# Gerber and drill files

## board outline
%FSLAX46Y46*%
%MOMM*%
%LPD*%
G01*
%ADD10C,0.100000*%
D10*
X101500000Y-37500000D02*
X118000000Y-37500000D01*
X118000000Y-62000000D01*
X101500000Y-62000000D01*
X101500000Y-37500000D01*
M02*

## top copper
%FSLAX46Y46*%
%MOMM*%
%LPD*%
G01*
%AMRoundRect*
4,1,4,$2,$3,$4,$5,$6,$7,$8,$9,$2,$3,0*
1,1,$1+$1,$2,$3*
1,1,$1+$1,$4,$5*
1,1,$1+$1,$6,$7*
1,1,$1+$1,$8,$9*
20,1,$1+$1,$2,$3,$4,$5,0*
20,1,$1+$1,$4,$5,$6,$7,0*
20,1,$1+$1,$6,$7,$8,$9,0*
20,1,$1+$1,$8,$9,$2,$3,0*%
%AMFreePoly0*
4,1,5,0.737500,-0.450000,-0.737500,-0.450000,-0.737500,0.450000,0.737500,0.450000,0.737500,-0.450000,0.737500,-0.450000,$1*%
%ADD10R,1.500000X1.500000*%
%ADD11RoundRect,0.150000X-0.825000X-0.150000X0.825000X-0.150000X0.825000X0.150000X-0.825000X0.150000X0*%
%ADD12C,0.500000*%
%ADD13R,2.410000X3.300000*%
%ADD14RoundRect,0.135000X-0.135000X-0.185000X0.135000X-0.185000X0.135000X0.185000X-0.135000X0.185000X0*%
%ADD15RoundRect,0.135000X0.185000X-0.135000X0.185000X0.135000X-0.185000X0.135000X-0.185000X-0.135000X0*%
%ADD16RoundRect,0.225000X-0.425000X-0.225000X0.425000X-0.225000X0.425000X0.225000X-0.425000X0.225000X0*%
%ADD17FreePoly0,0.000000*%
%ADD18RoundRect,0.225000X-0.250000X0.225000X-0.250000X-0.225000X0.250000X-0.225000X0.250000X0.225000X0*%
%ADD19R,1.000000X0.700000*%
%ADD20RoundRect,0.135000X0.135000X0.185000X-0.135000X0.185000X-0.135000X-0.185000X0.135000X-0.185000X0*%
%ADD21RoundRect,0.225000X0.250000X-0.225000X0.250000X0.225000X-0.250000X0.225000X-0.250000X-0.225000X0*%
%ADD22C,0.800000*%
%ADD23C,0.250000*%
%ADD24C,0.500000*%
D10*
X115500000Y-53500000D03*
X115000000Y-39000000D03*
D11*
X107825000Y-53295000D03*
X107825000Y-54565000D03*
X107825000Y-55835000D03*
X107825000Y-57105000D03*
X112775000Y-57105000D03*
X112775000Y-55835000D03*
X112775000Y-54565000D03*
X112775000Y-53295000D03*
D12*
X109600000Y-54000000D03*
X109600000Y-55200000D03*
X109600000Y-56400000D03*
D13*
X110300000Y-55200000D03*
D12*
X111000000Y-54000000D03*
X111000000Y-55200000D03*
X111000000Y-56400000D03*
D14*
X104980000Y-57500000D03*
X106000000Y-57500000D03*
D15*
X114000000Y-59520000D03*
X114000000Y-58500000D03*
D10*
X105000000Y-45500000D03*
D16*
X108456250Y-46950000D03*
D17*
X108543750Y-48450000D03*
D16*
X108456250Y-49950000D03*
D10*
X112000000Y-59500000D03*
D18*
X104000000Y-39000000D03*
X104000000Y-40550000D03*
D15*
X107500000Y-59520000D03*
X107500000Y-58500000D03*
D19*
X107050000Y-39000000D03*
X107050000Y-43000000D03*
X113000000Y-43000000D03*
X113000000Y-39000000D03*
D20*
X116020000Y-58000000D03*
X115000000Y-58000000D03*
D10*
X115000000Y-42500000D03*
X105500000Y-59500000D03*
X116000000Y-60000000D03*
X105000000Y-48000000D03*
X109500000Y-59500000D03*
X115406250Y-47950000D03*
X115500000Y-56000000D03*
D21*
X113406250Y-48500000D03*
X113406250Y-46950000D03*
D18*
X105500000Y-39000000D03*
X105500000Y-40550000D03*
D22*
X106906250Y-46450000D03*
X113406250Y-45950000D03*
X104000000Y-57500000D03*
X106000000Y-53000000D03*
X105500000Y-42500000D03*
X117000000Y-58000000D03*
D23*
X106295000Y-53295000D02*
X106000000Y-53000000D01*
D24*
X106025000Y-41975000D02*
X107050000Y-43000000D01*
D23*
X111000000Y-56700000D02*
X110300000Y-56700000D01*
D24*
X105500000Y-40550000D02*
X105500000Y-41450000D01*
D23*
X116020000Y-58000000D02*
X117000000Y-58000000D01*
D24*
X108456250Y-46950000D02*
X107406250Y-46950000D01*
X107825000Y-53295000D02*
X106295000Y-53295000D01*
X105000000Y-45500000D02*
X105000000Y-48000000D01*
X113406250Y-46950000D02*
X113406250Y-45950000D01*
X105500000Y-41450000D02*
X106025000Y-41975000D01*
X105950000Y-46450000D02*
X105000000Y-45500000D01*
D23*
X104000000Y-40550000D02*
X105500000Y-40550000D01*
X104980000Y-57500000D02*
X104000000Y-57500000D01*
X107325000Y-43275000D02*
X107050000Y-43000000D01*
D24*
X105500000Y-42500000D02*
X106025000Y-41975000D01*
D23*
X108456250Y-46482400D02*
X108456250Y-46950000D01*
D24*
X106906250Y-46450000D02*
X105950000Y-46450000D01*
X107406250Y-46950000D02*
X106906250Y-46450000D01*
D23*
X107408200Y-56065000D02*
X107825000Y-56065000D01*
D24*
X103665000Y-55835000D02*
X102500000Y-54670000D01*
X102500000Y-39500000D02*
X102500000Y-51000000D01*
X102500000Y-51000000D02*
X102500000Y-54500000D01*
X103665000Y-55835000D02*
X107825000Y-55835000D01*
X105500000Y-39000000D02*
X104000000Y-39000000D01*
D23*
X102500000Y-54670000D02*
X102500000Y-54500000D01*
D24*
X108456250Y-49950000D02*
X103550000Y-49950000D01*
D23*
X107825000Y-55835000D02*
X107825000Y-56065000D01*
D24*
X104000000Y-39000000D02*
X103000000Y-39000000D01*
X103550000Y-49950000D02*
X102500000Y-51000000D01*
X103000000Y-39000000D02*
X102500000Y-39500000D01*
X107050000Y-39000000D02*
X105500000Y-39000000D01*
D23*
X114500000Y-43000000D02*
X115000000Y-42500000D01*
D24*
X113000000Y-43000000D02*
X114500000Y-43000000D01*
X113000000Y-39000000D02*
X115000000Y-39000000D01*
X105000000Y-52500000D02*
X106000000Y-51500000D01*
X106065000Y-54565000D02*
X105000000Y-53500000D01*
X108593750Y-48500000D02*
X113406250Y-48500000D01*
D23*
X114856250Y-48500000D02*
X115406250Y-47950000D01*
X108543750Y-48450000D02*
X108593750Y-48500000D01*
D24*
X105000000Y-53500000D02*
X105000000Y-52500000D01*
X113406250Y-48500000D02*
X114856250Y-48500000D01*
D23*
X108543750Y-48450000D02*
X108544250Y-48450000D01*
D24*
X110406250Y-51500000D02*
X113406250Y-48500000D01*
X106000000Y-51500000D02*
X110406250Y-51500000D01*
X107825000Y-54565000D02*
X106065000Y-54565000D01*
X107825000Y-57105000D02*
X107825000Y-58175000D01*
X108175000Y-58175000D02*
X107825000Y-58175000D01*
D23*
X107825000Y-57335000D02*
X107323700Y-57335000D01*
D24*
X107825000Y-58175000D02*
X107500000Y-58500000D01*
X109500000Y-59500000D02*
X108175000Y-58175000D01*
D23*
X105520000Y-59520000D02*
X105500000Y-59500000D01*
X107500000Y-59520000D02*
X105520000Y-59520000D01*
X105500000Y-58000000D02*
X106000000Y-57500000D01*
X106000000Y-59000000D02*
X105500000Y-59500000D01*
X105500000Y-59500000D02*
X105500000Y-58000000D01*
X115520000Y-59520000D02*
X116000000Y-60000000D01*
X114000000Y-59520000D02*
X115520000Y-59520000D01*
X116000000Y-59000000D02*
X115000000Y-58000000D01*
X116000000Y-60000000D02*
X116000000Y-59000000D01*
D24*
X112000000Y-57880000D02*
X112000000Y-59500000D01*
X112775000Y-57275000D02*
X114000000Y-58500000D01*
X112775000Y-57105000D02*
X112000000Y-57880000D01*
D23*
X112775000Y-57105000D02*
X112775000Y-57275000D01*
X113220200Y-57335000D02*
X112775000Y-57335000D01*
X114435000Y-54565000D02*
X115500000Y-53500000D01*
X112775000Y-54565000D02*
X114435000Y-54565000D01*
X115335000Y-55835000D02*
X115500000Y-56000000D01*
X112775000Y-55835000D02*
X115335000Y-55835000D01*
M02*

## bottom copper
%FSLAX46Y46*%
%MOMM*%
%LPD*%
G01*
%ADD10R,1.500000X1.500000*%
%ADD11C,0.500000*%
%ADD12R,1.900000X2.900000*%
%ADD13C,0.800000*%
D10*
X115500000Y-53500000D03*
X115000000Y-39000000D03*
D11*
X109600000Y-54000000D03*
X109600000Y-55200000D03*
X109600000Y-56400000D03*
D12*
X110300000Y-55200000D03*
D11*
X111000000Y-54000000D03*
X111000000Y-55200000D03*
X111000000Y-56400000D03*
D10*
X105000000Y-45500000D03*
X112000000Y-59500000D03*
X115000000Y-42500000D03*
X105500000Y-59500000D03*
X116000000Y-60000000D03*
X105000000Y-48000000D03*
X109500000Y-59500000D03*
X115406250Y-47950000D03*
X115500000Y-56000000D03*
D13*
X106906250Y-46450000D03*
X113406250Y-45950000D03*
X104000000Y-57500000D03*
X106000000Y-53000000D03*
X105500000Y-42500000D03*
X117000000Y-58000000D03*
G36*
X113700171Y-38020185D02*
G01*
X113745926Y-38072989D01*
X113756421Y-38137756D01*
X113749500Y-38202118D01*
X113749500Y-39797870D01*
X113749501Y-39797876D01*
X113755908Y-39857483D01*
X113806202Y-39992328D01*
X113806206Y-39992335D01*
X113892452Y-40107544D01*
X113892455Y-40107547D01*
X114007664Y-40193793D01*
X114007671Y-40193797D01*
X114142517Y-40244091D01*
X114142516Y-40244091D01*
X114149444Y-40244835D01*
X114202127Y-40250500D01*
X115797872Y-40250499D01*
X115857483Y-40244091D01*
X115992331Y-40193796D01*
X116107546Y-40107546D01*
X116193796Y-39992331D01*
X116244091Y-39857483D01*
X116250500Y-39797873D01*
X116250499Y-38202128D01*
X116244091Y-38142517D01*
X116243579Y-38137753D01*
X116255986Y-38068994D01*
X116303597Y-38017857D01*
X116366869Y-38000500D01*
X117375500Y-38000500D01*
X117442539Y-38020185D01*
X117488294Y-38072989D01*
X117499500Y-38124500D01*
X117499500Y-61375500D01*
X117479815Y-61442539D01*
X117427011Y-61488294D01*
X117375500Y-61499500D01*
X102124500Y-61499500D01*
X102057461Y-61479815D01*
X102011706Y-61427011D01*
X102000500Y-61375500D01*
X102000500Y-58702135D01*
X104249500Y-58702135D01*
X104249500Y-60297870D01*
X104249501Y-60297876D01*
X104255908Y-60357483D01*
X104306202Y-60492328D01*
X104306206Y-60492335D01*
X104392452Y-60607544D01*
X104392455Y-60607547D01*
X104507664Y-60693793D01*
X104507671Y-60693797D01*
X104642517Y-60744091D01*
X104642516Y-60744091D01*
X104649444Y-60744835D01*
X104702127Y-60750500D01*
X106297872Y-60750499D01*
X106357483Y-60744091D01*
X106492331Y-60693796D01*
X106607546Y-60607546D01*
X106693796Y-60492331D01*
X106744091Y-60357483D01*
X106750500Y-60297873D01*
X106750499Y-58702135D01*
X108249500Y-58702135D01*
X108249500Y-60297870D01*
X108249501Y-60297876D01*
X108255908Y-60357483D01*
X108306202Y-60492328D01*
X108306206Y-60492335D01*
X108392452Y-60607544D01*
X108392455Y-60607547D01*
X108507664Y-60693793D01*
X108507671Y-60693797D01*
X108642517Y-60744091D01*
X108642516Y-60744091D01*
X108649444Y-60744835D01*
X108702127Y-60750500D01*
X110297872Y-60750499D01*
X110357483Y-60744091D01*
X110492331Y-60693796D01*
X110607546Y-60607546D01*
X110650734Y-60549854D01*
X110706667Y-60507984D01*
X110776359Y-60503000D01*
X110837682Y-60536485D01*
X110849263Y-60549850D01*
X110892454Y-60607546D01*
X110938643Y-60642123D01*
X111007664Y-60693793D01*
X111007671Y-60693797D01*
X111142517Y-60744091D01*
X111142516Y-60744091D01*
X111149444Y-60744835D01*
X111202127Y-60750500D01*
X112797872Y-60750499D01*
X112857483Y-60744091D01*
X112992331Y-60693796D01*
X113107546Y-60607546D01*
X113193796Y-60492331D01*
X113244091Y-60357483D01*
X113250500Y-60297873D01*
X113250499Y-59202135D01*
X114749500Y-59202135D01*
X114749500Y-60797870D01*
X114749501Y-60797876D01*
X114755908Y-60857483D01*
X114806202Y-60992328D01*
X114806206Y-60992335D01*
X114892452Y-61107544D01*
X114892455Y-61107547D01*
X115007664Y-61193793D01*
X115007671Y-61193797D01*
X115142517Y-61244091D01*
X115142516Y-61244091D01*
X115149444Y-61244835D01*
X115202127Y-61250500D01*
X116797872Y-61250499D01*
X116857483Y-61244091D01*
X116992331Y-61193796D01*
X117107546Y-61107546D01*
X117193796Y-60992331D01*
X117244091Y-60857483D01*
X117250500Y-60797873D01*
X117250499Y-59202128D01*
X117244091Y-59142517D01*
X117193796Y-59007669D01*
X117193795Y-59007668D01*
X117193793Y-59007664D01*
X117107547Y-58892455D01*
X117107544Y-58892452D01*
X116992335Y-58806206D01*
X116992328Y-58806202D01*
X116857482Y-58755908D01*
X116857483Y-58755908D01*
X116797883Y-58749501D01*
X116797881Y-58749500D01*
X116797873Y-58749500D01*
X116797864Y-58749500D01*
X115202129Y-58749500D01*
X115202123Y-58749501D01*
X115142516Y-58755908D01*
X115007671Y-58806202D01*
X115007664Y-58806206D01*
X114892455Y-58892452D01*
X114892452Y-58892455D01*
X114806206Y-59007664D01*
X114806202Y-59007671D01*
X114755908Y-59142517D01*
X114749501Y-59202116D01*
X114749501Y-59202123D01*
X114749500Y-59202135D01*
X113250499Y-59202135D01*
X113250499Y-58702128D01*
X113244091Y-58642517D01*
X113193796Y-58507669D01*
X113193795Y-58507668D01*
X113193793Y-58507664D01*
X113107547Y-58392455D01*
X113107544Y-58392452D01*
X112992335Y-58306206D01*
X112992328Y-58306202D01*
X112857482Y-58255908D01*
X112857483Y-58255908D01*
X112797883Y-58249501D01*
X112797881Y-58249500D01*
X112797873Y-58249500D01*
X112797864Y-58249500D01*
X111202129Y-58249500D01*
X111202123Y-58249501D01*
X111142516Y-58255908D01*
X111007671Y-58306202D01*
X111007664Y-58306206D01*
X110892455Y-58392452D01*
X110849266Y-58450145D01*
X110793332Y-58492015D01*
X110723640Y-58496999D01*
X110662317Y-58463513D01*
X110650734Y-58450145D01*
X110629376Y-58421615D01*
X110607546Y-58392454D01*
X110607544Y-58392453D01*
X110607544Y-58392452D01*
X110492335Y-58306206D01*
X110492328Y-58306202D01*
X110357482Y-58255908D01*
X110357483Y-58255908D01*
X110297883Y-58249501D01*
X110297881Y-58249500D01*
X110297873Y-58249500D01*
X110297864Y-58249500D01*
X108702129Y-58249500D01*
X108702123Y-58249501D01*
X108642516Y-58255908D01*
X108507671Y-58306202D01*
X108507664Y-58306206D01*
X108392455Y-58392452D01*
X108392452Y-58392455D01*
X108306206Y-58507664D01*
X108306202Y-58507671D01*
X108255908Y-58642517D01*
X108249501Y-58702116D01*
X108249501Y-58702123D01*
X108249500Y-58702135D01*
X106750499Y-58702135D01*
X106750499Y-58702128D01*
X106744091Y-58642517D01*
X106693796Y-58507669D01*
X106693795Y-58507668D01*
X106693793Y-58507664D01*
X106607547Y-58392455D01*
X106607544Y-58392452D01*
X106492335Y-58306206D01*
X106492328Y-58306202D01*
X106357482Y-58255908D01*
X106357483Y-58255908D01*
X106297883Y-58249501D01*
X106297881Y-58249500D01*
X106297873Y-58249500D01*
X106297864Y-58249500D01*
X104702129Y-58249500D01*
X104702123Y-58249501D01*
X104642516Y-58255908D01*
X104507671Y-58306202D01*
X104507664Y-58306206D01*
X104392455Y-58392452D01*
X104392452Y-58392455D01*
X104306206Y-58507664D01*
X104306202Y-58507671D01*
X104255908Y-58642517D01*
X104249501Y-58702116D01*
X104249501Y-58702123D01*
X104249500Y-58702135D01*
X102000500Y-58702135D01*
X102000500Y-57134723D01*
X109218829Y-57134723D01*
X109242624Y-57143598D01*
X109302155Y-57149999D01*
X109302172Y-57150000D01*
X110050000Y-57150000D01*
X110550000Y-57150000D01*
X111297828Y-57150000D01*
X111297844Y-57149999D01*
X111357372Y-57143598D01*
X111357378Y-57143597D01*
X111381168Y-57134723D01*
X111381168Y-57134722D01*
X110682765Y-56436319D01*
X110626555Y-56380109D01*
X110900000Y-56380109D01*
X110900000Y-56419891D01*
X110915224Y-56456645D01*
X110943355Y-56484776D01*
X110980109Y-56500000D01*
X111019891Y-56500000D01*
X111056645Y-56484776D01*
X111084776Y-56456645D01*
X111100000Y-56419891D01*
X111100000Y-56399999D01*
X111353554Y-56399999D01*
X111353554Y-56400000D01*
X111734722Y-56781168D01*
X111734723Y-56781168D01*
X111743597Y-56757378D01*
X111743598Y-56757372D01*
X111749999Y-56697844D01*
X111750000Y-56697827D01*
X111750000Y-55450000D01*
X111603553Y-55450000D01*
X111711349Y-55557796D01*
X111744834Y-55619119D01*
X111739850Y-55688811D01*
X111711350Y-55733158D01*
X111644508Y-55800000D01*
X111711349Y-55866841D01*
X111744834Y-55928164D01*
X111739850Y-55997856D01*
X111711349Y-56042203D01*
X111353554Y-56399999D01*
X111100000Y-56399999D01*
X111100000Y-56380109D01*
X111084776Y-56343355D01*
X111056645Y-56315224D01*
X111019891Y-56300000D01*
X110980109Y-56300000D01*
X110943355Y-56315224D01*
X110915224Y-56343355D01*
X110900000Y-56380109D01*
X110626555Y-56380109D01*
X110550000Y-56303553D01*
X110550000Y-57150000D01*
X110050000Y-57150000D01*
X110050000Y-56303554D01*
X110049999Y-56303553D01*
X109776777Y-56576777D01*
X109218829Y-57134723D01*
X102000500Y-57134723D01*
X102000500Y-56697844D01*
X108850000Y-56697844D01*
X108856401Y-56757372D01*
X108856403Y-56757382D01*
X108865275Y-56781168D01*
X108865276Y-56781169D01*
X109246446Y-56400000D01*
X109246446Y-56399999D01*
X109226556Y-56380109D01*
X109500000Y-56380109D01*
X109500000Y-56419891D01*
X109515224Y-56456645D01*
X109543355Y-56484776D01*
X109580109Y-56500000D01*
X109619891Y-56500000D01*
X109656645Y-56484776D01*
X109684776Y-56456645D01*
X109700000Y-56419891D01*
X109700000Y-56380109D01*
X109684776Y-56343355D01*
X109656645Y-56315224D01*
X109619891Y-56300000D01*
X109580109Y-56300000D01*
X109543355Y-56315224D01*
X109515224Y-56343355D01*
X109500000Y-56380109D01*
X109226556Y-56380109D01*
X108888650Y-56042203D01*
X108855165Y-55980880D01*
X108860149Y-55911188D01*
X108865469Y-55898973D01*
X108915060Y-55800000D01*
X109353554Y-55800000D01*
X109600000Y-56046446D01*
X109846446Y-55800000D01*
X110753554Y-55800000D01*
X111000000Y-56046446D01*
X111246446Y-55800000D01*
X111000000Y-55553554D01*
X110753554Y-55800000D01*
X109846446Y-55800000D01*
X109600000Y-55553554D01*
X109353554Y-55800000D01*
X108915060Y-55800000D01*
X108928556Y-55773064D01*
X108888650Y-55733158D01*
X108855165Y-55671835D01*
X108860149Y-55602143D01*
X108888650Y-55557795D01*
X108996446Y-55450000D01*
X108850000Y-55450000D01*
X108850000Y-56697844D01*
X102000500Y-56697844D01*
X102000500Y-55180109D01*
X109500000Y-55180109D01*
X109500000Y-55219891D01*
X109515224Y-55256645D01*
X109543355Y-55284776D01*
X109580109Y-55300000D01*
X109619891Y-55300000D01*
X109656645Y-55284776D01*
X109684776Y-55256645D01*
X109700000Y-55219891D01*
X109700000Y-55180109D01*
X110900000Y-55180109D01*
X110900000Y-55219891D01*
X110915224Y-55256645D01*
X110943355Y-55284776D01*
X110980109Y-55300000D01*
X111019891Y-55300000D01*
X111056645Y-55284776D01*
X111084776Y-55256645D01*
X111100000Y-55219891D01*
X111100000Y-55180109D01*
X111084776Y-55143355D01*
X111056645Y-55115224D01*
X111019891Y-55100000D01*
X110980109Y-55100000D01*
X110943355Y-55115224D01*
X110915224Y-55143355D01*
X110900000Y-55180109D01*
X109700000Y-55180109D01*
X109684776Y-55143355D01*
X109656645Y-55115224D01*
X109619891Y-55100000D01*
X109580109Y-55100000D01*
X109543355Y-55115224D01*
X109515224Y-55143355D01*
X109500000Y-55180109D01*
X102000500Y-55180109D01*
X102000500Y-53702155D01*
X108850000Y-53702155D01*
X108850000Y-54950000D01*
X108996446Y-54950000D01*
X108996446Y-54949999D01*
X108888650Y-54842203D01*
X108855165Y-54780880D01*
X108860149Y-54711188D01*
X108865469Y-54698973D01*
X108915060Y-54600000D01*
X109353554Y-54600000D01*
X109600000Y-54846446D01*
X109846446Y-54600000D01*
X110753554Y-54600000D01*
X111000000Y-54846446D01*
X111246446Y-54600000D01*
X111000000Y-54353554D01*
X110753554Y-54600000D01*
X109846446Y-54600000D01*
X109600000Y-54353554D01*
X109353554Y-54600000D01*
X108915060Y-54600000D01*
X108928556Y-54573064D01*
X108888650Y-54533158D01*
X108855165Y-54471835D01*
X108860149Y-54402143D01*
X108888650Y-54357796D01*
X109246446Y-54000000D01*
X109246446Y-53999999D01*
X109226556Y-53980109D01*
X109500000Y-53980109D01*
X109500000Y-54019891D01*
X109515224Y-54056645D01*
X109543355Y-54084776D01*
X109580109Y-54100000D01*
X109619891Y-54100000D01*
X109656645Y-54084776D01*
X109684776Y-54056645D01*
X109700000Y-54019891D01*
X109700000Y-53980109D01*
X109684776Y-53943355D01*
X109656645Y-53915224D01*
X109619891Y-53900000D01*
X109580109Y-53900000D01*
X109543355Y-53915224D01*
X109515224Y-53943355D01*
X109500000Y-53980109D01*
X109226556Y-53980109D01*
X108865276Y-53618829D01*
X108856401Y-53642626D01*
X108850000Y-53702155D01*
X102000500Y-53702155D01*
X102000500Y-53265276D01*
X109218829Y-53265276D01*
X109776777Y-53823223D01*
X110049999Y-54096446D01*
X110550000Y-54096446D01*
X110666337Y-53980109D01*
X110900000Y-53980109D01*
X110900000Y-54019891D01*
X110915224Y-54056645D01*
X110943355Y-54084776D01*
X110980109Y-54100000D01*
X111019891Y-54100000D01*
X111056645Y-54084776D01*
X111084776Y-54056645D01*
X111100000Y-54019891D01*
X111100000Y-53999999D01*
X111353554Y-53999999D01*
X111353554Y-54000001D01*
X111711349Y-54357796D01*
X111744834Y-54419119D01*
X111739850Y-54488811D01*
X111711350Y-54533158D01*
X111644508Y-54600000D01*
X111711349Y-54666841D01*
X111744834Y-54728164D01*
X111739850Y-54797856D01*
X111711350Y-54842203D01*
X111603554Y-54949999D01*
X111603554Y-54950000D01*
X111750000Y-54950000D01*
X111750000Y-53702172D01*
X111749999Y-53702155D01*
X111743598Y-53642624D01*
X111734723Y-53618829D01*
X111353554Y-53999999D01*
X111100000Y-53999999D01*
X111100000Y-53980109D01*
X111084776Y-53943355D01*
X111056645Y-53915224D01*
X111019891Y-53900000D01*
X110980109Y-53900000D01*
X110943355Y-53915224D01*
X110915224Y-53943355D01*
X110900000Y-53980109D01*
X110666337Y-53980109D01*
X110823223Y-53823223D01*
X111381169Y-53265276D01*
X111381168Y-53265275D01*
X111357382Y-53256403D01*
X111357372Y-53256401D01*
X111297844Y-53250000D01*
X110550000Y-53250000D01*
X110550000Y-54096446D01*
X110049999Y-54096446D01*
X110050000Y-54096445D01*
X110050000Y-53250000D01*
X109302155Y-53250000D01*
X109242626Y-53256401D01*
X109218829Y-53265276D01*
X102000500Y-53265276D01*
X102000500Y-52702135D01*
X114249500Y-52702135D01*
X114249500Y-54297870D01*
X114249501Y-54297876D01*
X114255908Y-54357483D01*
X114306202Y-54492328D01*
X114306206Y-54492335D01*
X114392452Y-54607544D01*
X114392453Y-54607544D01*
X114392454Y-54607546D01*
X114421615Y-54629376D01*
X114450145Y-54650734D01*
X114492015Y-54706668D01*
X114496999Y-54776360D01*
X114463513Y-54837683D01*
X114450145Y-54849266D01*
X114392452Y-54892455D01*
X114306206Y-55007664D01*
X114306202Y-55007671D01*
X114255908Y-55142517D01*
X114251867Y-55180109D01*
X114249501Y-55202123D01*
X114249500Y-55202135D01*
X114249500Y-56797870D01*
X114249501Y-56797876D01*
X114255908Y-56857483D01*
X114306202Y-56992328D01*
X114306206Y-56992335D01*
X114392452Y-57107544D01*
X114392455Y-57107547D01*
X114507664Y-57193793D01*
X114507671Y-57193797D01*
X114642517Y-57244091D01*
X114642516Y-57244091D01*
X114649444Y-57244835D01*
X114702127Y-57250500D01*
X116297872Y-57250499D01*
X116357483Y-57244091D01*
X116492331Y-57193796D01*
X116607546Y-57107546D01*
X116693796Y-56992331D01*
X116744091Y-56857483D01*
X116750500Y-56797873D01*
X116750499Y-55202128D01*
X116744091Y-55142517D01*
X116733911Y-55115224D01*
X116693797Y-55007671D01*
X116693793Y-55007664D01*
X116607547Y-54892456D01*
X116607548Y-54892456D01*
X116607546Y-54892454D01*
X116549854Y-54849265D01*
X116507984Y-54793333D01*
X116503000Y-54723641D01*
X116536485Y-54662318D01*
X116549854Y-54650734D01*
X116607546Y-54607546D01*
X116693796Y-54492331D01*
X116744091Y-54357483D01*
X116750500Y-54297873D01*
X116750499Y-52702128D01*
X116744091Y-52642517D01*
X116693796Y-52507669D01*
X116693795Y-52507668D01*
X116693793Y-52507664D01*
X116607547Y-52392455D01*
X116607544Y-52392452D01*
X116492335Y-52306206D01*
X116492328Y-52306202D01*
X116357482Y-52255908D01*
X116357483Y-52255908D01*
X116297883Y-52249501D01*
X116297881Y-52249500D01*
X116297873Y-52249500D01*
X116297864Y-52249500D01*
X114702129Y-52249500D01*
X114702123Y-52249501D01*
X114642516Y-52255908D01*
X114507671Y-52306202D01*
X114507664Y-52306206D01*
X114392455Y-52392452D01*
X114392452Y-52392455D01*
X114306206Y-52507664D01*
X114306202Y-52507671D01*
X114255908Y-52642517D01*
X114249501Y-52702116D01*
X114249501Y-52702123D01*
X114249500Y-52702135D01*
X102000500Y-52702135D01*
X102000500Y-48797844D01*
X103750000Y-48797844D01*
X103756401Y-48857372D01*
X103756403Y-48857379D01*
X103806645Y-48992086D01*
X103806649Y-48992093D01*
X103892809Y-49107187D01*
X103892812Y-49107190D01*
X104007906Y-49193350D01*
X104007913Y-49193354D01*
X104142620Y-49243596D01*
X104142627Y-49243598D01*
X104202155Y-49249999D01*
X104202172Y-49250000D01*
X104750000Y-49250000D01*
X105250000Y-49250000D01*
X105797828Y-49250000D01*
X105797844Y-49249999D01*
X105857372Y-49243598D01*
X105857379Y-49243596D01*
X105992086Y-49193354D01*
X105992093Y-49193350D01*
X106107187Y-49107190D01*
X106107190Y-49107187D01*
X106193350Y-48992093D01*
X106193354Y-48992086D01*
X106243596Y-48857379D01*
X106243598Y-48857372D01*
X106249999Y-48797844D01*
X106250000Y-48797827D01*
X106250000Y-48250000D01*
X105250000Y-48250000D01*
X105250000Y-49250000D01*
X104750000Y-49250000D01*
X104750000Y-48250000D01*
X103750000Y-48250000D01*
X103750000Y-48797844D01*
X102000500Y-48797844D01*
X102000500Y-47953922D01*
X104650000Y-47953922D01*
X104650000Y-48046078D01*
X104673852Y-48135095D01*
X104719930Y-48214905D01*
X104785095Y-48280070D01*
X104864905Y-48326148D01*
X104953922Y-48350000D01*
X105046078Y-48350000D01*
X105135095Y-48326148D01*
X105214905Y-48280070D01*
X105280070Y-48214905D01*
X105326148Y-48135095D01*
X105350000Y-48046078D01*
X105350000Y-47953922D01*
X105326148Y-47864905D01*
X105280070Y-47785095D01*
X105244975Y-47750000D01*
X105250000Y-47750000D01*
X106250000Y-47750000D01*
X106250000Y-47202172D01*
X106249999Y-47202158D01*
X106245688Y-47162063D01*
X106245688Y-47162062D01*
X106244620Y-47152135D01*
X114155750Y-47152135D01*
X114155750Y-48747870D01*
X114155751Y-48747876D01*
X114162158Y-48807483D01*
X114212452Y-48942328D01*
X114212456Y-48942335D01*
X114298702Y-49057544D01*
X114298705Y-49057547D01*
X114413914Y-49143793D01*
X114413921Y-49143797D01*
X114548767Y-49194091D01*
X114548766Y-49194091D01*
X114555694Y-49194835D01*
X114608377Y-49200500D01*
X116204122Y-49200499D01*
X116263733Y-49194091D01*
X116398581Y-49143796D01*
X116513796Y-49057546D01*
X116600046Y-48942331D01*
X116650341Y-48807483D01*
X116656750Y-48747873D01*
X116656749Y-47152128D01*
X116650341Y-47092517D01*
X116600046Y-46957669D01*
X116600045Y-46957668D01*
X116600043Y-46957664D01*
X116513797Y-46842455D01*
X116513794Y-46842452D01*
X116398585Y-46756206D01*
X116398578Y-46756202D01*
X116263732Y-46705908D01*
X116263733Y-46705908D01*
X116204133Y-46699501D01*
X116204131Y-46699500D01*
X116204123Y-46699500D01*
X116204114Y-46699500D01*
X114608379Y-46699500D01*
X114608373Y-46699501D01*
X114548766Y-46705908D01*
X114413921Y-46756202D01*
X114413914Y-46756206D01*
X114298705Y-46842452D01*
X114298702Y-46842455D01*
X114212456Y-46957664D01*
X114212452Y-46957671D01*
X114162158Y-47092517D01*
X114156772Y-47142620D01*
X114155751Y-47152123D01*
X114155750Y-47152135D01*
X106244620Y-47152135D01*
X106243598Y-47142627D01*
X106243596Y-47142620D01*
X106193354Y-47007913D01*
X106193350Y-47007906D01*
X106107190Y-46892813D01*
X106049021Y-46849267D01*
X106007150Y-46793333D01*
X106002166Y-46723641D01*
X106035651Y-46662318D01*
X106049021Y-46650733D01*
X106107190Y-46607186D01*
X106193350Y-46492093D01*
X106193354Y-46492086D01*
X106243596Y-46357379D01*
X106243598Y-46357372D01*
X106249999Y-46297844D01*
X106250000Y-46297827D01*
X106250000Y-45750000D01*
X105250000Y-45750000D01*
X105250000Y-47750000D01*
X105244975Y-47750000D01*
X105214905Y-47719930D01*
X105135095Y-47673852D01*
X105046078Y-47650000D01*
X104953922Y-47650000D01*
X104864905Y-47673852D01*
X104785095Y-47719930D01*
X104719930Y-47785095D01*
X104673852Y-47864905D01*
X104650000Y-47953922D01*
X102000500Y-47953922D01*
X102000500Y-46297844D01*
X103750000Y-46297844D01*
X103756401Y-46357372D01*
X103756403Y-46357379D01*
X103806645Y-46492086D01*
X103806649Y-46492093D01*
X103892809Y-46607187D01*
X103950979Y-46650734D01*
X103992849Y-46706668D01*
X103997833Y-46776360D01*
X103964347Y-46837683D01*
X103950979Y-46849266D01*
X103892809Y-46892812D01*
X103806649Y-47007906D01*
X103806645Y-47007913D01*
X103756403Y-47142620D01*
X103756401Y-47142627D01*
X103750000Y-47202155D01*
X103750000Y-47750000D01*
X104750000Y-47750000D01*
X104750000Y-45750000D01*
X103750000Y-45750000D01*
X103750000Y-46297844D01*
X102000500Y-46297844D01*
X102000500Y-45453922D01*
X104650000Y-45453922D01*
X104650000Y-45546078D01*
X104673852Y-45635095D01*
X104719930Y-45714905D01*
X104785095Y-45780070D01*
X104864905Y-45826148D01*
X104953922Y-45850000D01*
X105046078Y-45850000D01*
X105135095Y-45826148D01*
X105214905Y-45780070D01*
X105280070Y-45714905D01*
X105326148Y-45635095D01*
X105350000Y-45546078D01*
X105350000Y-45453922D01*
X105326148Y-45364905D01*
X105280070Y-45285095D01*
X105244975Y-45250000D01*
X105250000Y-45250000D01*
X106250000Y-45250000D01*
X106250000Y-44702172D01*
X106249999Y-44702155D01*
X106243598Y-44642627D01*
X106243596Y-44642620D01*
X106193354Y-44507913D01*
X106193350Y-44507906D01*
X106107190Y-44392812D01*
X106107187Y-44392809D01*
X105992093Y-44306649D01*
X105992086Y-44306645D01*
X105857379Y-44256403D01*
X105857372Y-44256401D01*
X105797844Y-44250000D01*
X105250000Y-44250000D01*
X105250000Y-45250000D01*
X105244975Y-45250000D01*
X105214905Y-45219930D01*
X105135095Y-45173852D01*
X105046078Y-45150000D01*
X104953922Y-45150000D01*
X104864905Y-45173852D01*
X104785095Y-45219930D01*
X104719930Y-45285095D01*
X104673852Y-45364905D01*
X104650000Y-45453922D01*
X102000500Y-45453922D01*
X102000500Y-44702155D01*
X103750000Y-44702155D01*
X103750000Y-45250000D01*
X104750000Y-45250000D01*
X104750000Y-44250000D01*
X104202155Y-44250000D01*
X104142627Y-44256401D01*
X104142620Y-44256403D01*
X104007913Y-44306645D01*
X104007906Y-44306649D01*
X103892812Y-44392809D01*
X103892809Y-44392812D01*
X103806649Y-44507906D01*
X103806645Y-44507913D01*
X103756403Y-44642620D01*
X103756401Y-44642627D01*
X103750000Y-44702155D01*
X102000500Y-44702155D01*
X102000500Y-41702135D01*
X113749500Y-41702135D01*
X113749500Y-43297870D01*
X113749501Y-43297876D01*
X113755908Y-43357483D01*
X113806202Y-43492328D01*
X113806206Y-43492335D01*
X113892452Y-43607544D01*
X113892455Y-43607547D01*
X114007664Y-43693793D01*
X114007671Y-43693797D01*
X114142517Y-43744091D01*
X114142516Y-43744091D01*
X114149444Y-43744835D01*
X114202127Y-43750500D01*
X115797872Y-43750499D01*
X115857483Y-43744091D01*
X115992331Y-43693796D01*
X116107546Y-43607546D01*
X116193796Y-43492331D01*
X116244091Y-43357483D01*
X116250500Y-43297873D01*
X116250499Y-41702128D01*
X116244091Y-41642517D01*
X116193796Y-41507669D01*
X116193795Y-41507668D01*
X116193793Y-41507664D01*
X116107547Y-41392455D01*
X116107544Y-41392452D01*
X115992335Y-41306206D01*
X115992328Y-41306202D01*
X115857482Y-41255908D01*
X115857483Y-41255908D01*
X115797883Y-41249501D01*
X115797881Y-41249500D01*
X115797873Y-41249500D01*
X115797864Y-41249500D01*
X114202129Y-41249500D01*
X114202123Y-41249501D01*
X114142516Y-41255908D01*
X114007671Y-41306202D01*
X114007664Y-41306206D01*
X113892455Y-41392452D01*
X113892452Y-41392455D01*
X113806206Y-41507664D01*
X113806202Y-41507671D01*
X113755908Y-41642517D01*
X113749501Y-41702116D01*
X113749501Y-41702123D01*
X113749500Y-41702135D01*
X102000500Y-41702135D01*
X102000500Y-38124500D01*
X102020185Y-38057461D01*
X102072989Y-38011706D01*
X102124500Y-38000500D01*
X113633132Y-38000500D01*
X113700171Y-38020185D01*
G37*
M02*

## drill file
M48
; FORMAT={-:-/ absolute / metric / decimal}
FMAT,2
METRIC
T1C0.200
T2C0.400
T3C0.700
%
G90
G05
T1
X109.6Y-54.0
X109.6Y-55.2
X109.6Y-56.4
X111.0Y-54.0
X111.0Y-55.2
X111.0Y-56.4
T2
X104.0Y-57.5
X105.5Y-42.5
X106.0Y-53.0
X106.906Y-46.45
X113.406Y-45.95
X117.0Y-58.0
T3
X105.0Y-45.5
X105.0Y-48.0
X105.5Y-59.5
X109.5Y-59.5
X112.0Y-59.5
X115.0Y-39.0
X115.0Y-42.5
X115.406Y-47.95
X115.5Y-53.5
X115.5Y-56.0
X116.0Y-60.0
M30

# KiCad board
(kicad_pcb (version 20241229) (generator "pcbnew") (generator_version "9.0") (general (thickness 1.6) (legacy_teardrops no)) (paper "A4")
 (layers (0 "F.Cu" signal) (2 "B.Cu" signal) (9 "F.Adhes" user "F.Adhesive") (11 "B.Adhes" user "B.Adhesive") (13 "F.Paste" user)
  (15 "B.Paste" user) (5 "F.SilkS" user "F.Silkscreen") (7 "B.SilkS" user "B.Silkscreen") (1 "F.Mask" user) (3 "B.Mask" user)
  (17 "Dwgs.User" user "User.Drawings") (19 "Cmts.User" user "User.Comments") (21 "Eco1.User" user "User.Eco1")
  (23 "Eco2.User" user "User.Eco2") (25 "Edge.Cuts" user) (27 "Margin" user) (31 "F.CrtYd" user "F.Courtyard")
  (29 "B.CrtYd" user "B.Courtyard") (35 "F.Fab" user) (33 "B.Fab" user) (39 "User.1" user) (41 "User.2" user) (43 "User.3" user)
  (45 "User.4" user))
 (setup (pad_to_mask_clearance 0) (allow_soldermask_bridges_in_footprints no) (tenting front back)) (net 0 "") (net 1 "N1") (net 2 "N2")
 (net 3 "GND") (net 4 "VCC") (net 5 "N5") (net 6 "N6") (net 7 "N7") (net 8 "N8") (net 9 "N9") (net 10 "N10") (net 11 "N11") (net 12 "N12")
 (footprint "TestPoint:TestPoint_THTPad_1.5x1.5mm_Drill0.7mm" (layer "F.Cu") (at 115.5 53.5)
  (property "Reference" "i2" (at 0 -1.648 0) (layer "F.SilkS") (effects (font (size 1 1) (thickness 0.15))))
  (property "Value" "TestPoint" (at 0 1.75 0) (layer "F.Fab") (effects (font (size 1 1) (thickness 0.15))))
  (pad "1" thru_hole rect (at 0 0) (size 1.5 1.5) (drill 0.7) (layers "*.Cu" "*.Mask") (remove_unused_layers no) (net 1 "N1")))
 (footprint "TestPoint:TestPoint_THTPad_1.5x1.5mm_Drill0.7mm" (layer "F.Cu") (at 115 39)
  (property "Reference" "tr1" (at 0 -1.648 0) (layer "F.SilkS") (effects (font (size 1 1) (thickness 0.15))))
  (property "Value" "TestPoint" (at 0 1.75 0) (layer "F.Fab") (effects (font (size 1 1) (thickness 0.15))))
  (pad "1" thru_hole rect (at 0 0) (size 1.5 1.5) (drill 0.7) (layers "*.Cu" "*.Mask") (remove_unused_layers no) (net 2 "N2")))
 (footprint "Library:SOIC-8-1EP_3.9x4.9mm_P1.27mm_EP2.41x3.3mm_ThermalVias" (layer "F.Cu") (at 110.3 55.2)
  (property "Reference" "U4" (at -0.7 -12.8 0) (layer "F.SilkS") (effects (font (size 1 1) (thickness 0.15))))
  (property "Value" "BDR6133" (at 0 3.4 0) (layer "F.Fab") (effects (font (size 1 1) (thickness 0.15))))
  (pad "" smd roundrect (at -0.6 -0.825) (size 1.01 1.38) (layers "F.Paste") (roundrect_rratio 0.247525))
  (pad "" smd roundrect (at -0.6 0.825) (size 1.01 1.38) (layers "F.Paste") (roundrect_rratio 0.247525))
  (pad "" smd roundrect (at 0.6 -0.825) (size 1.01 1.38) (layers "F.Paste") (roundrect_rratio 0.247525))
  (pad "" smd roundrect (at 0.6 0.825) (size 1.01 1.38) (layers "F.Paste") (roundrect_rratio 0.247525))
  (pad "1" smd roundrect (at -2.475 -1.905) (size 1.95 0.6) (layers "F.Cu" "F.Mask" "F.Paste") (roundrect_rratio 0.25) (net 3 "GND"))
  (pad "2" smd roundrect (at -2.475 -0.635) (size 1.95 0.6) (layers "F.Cu" "F.Mask" "F.Paste") (roundrect_rratio 0.25) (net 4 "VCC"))
  (pad "3" smd roundrect (at -2.475 0.635) (size 1.95 0.6) (layers "F.Cu" "F.Mask" "F.Paste") (roundrect_rratio 0.25) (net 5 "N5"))
  (pad "4" smd roundrect (at -2.475 1.905) (size 1.95 0.6) (layers "F.Cu" "F.Mask" "F.Paste") (roundrect_rratio 0.25) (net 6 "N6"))
  (pad "5" smd roundrect (at 2.475 1.905) (size 1.95 0.6) (layers "F.Cu" "F.Mask" "F.Paste") (roundrect_rratio 0.25) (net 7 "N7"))
  (pad "6" smd roundrect (at 2.475 0.635) (size 1.95 0.6) (layers "F.Cu" "F.Mask" "F.Paste") (roundrect_rratio 0.25) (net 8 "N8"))
  (pad "7" smd roundrect (at 2.475 -0.635) (size 1.95 0.6) (layers "F.Cu" "F.Mask" "F.Paste") (roundrect_rratio 0.25) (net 1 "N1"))
  (pad "8" smd roundrect (at 2.475 -1.905) (size 1.95 0.6) (layers "F.Cu" "F.Mask" "F.Paste") (roundrect_rratio 0.25) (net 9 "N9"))
  (pad "9" thru_hole circle (at -0.7 -1.2) (size 0.5 0.5) (drill 0.2) (layers "*.Cu") (remove_unused_layers no) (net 3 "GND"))
  (pad "9" thru_hole circle (at -0.7 0) (size 0.5 0.5) (drill 0.2) (layers "*.Cu") (remove_unused_layers no) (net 3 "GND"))
  (pad "9" thru_hole circle (at -0.7 1.2) (size 0.5 0.5) (drill 0.2) (layers "*.Cu") (remove_unused_layers no) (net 3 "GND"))
  (pad "9" smd rect (at 0 0) (size 1.9 2.9) (layers "B.Cu") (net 3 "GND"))
  (pad "9" smd rect (at 0 0) (size 2.41 3.3) (layers "F.Cu" "F.Mask") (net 3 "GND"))
  (pad "9" thru_hole circle (at 0.7 -1.2) (size 0.5 0.5) (drill 0.2) (layers "*.Cu") (remove_unused_layers no) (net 3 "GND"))
  (pad "9" thru_hole circle (at 0.7 0) (size 0.5 0.5) (drill 0.2) (layers "*.Cu") (remove_unused_layers no) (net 3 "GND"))
  (pad "9" thru_hole circle (at 0.7 1.2) (size 0.5 0.5) (drill 0.2) (layers "*.Cu") (remove_unused_layers no) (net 3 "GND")))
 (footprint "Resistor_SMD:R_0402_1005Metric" (layer "F.Cu") (at 105.49 57.5)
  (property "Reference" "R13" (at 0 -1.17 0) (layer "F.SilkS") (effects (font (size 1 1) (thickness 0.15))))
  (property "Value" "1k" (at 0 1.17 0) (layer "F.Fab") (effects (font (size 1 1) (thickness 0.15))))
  (pad "1" smd roundrect (at -0.51 0) (size 0.54 0.64) (layers "F.Cu" "F.Mask" "F.Paste") (roundrect_rratio 0.25) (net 3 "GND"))
  (pad "2" smd roundrect (at 0.51 0) (size 0.54 0.64) (layers "F.Cu" "F.Mask" "F.Paste") (roundrect_rratio 0.25) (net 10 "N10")))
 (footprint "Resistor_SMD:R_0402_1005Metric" (layer "F.Cu") (at 114 59.01 90)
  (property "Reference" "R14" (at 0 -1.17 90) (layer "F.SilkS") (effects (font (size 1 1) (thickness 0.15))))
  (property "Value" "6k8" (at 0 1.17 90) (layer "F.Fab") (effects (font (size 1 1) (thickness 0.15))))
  (pad "1" smd roundrect (at -0.51 0 90) (size 0.54 0.64) (layers "F.Cu" "F.Mask" "F.Paste") (roundrect_rratio 0.25) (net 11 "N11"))
  (pad "2" smd roundrect (at 0.51 0 90) (size 0.54 0.64) (layers "F.Cu" "F.Mask" "F.Paste") (roundrect_rratio 0.25) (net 7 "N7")))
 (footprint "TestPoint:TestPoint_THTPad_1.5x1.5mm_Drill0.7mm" (layer "F.Cu") (at 105 45.5)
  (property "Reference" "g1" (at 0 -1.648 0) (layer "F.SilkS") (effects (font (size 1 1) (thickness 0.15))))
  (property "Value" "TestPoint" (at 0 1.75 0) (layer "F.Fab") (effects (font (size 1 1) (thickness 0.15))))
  (pad "1" thru_hole rect (at 0 0) (size 1.5 1.5) (drill 0.7) (layers "*.Cu" "*.Mask") (remove_unused_layers no) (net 3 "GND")))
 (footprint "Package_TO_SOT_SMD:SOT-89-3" (layer "F.Cu") (at 110.40625 48.45)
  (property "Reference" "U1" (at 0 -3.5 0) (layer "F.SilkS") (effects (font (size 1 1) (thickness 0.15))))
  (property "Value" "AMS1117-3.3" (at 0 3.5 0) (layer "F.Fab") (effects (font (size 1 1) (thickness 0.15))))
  (pad "1" smd roundrect (at -1.95 -1.5) (size 1.3 0.9) (layers "F.Cu" "F.Mask" "F.Paste") (roundrect_rratio 0.25) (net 3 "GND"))
  (pad "2" smd custom (at -1.8625 0) (size 1.475 0.9) (layers "F.Cu" "F.Mask" "F.Paste") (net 4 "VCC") (zone_connect 2)
   (thermal_bridge_angle 45) (options (clearance outline) (anchor rect)) (primitives))
  (pad "3" smd roundrect (at -1.95 1.5) (size 1.3 0.9) (layers "F.Cu" "F.Mask" "F.Paste") (roundrect_rratio 0.25) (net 5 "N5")))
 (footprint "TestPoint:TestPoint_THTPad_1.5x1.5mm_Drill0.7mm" (layer "F.Cu") (at 112 59.5)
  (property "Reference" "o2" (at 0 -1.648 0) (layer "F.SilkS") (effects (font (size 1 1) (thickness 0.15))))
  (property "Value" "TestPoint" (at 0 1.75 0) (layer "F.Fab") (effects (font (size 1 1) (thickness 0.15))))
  (pad "1" thru_hole rect (at 0 0) (size 1.5 1.5) (drill 0.7) (layers "*.Cu" "*.Mask") (remove_unused_layers no) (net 7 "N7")))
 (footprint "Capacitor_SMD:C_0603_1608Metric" (layer "F.Cu") (at 104 39.775 -90)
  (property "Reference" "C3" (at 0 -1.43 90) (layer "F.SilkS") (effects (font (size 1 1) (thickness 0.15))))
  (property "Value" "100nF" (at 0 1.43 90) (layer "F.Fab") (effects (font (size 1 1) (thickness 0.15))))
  (pad "1" smd roundrect (at -0.775 0 270) (size 0.9 0.95) (layers "F.Cu" "F.Mask" "F.Paste") (roundrect_rratio 0.25) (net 5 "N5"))
  (pad "2" smd roundrect (at 0.775 0 270) (size 0.9 0.95) (layers "F.Cu" "F.Mask" "F.Paste") (roundrect_rratio 0.25) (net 3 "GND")))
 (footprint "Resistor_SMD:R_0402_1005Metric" (layer "F.Cu") (at 107.5 59.01 90)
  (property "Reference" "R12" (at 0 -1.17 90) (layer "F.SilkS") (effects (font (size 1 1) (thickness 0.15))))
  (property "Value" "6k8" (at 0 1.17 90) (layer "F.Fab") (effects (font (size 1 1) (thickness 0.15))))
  (pad "1" smd roundrect (at -0.51 0 90) (size 0.54 0.64) (layers "F.Cu" "F.Mask" "F.Paste") (roundrect_rratio 0.25) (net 10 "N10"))
  (pad "2" smd roundrect (at 0.51 0 90) (size 0.54 0.64) (layers "F.Cu" "F.Mask" "F.Paste") (roundrect_rratio 0.25) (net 6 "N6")))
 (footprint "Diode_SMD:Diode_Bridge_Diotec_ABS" (layer "F.Cu") (at 110.025 41)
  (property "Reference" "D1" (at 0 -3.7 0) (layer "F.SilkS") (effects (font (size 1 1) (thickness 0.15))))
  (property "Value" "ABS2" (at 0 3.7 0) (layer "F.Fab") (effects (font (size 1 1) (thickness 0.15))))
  (pad "1" smd rect (at -2.975 -2) (size 1 0.7) (layers "F.Cu" "F.Mask" "F.Paste") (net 5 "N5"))
  (pad "2" smd rect (at -2.975 2) (size 1 0.7) (layers "F.Cu" "F.Mask" "F.Paste") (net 3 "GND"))
  (pad "3" smd rect (at 2.975 2) (size 1 0.7) (layers "F.Cu" "F.Mask" "F.Paste") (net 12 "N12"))
  (pad "4" smd rect (at 2.975 -2) (size 1 0.7) (layers "F.Cu" "F.Mask" "F.Paste") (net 2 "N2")))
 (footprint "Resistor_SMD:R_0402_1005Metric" (layer "F.Cu") (at 115.51 58 180)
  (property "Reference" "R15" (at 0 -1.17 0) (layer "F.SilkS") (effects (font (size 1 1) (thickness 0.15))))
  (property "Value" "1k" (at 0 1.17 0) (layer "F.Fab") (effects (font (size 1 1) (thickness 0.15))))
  (pad "1" smd roundrect (at -0.51 0 180) (size 0.54 0.64) (layers "F.Cu" "F.Mask" "F.Paste") (roundrect_rratio 0.25) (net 3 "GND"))
  (pad "2" smd roundrect (at 0.51 0 180) (size 0.54 0.64) (layers "F.Cu" "F.Mask" "F.Paste") (roundrect_rratio 0.25) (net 11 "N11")))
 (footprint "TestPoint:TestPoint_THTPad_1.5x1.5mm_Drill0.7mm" (layer "F.Cu") (at 115 42.5)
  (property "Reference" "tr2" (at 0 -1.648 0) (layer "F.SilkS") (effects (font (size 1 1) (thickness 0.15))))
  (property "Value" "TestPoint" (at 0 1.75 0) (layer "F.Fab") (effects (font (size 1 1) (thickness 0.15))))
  (pad "1" thru_hole rect (at 0 0) (size 1.5 1.5) (drill 0.7) (layers "*.Cu" "*.Mask") (remove_unused_layers no) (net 12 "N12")))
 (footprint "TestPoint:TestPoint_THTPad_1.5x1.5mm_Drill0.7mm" (layer "F.Cu") (at 105.5 59.5)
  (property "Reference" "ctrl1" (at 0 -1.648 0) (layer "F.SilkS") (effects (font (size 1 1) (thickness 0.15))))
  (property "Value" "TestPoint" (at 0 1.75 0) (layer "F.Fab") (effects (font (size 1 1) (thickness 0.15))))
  (pad "1" thru_hole rect (at 0 0) (size 1.5 1.5) (drill 0.7) (layers "*.Cu" "*.Mask") (remove_unused_layers no) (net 10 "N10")))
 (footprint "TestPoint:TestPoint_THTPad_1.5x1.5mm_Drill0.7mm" (layer "F.Cu") (at 116 60)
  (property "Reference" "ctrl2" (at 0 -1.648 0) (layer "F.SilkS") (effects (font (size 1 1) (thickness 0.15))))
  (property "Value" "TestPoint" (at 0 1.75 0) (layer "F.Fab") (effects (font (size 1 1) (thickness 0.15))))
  (pad "1" thru_hole rect (at 0 0) (size 1.5 1.5) (drill 0.7) (layers "*.Cu" "*.Mask") (remove_unused_layers no) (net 11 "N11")))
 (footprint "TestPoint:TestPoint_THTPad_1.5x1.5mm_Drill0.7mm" (layer "F.Cu") (at 105 48)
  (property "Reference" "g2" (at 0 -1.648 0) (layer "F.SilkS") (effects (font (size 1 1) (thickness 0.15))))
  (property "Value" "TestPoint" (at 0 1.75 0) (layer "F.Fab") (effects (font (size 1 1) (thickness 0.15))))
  (pad "1" thru_hole rect (at 0 0) (size 1.5 1.5) (drill 0.7) (layers "*.Cu" "*.Mask") (remove_unused_layers no) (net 3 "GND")))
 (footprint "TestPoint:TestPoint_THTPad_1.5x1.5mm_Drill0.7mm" (layer "F.Cu") (at 109.5 59.5)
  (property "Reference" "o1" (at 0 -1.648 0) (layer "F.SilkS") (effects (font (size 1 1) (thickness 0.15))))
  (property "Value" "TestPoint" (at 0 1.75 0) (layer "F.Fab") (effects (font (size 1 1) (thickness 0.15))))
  (pad "1" thru_hole rect (at 0 0) (size 1.5 1.5) (drill 0.7) (layers "*.Cu" "*.Mask") (remove_unused_layers no) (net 6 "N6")))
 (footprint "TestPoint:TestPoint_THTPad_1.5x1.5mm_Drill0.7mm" (layer "F.Cu") (at 115.40625 47.95)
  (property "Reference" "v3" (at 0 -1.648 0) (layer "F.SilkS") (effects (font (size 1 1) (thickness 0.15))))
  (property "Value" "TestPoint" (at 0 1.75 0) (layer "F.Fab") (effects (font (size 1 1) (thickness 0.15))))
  (pad "1" thru_hole rect (at 0 0) (size 1.5 1.5) (drill 0.7) (layers "*.Cu" "*.Mask") (remove_unused_layers no) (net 4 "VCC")))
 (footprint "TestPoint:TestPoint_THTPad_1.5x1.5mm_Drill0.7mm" (layer "F.Cu") (at 115.5 56)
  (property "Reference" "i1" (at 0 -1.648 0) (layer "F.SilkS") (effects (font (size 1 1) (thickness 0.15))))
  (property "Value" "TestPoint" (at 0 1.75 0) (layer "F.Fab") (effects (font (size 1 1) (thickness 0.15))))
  (pad "1" thru_hole rect (at 0 0) (size 1.5 1.5) (drill 0.7) (layers "*.Cu" "*.Mask") (remove_unused_layers no) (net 8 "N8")))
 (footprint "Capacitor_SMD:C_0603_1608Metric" (layer "F.Cu") (at 113.40625 47.725 90)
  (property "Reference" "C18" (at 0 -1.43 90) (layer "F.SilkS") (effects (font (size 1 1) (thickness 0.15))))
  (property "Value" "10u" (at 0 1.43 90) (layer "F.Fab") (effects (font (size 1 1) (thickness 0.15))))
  (pad "1" smd roundrect (at -0.775 0 90) (size 0.9 0.95) (layers "F.Cu" "F.Mask" "F.Paste") (roundrect_rratio 0.25) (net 4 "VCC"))
  (pad "2" smd roundrect (at 0.775 0 90) (size 0.9 0.95) (layers "F.Cu" "F.Mask" "F.Paste") (roundrect_rratio 0.25) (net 3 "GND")))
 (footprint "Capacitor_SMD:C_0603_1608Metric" (layer "F.Cu") (at 105.5 39.775 -90)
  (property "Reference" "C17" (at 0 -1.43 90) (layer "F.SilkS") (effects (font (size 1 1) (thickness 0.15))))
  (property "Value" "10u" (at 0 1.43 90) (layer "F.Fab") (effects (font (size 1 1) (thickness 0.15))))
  (pad "1" smd roundrect (at -0.775 0 270) (size 0.9 0.95) (layers "F.Cu" "F.Mask" "F.Paste") (roundrect_rratio 0.25) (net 5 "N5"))
  (pad "2" smd roundrect (at 0.775 0 270) (size 0.9 0.95) (layers "F.Cu" "F.Mask" "F.Paste") (roundrect_rratio 0.25) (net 3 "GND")))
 (gr_rect (start 101.5 37.5) (end 118 62) (stroke (width 0.1) (type default)) (fill no) (layer "Edge.Cuts"))
 (segment (start 106.295 53.295) (end 106 53) (width 0.25) (layer "F.Cu") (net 3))
 (segment (start 106.025 41.975) (end 107.05 43) (width 0.5) (layer "F.Cu") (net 3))
 (segment (start 111 56.7) (end 110.3 56.7) (width 0.25) (layer "F.Cu") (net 3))
 (segment (start 105.5 40.55) (end 105.5 41.45) (width 0.5) (layer "F.Cu") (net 3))
 (segment (start 116.02 58) (end 117 58) (width 0.25) (layer "F.Cu") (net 3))
 (segment (start 108.45625 46.95) (end 107.40625 46.95) (width 0.5) (layer "F.Cu") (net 3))
 (segment (start 107.825 53.295) (end 106.295 53.295) (width 0.5) (layer "F.Cu") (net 3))
 (segment (start 105 45.5) (end 105 48) (width 0.5) (layer "F.Cu") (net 3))
 (segment (start 113.40625 46.95) (end 113.40625 45.95) (width 0.5) (layer "F.Cu") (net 3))
 (segment (start 105.5 41.45) (end 106.025 41.975) (width 0.5) (layer "F.Cu") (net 3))
 (segment (start 105.95 46.45) (end 105 45.5) (width 0.5) (layer "F.Cu") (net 3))
 (segment (start 104 40.55) (end 105.5 40.55) (width 0.25) (layer "F.Cu") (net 3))
 (segment (start 104.98 57.5) (end 104 57.5) (width 0.25) (layer "F.Cu") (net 3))
 (segment (start 107.325 43.275) (end 107.05 43) (width 0.25) (layer "F.Cu") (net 3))
 (segment (start 105.5 42.5) (end 106.025 41.975) (width 0.5) (layer "F.Cu") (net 3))
 (segment (start 108.45625 46.4824) (end 108.45625 46.95) (width 0.25) (layer "F.Cu") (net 3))
 (segment (start 106.90625 46.45) (end 105.95 46.45) (width 0.5) (layer "F.Cu") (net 3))
 (segment (start 107.40625 46.95) (end 106.90625 46.45) (width 0.5) (layer "F.Cu") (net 3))
 (via (at 106.90625 46.45) (size 0.8) (drill 0.4) (layers "F.Cu" "B.Cu") (free yes) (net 3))
 (via (at 113.40625 45.95) (size 0.8) (drill 0.4) (layers "F.Cu" "B.Cu") (free yes) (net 3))
 (via (at 104 57.5) (size 0.8) (drill 0.4) (layers "F.Cu" "B.Cu") (free yes) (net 3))
 (via (at 106 53) (size 0.8) (drill 0.4) (layers "F.Cu" "B.Cu") (free yes) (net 3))
 (via (at 105.5 42.5) (size 0.8) (drill 0.4) (layers "F.Cu" "B.Cu") (free yes) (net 3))
 (via (at 117 58) (size 0.8) (drill 0.4) (layers "F.Cu" "B.Cu") (free yes) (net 3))
 (segment (start 107.4082 56.065) (end 107.825 56.065) (width 0.25) (layer "F.Cu") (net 5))
 (segment (start 103.665 55.835) (end 102.5 54.67) (width 0.5) (layer "F.Cu") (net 5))
 (segment (start 102.5 39.5) (end 102.5 51) (width 0.5) (layer "F.Cu") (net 5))
 (segment (start 102.5 51) (end 102.5 54.5) (width 0.5) (layer "F.Cu") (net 5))
 (segment (start 103.665 55.835) (end 107.825 55.835) (width 0.5) (layer "F.Cu") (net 5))
 (segment (start 105.5 39) (end 104 39) (width 0.5) (layer "F.Cu") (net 5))
 (segment (start 102.5 54.67) (end 102.5 54.5) (width 0.25) (layer "F.Cu") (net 5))
 (segment (start 108.45625 49.95) (end 103.55 49.95) (width 0.5) (layer "F.Cu") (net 5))
 (segment (start 107.825 55.835) (end 107.825 56.065) (width 0.25) (layer "F.Cu") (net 5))
 (segment (start 104 39) (end 103 39) (width 0.5) (layer "F.Cu") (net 5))
 (segment (start 103.55 49.95) (end 102.5 51) (width 0.5) (layer "F.Cu") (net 5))
 (segment (start 103 39) (end 102.5 39.5) (width 0.5) (layer "F.Cu") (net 5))
 (segment (start 107.05 39) (end 105.5 39) (width 0.5) (layer "F.Cu") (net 5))
 (segment (start 114.5 43) (end 115 42.5) (width 0.25) (layer "F.Cu") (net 12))
 (segment (start 113 43) (end 114.5 43) (width 0.5) (layer "F.Cu") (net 12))
 (segment (start 113 39) (end 115 39) (width 0.5) (layer "F.Cu") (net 2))
 (segment (start 105 52.5) (end 106 51.5) (width 0.5) (layer "F.Cu") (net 4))
 (segment (start 106.065 54.565) (end 105 53.5) (width 0.5) (layer "F.Cu") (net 4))
 (segment (start 108.59375 48.5) (end 113.40625 48.5) (width 0.5) (layer "F.Cu") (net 4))
 (segment (start 114.85625 48.5) (end 115.40625 47.95) (width 0.25) (layer "F.Cu") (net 4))
 (segment (start 108.54375 48.45) (end 108.59375 48.5) (width 0.25) (layer "F.Cu") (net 4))
 (segment (start 105 53.5) (end 105 52.5) (width 0.5) (layer "F.Cu") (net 4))
 (segment (start 113.40625 48.5) (end 114.85625 48.5) (width 0.5) (layer "F.Cu") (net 4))
 (segment (start 108.54375 48.45) (end 108.54425 48.45) (width 0.25) (layer "F.Cu") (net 4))
 (segment (start 110.40625 51.5) (end 113.40625 48.5) (width 0.5) (layer "F.Cu") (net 4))
 (segment (start 106 51.5) (end 110.40625 51.5) (width 0.5) (layer "F.Cu") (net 4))
 (segment (start 107.825 54.565) (end 106.065 54.565) (width 0.5) (layer "F.Cu") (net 4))
 (segment (start 107.825 57.105) (end 107.825 58.175) (width 0.5) (layer "F.Cu") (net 6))
 (segment (start 108.175 58.175) (end 107.825 58.175) (width 0.5) (layer "F.Cu") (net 6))
 (segment (start 107.825 57.335) (end 107.3237 57.335) (width 0.25) (layer "F.Cu") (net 6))
 (segment (start 107.825 58.175) (end 107.5 58.5) (width 0.5) (layer "F.Cu") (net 6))
 (segment (start 109.5 59.5) (end 108.175 58.175) (width 0.5) (layer "F.Cu") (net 6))
 (segment (start 105.52 59.52) (end 105.5 59.5) (width 0.25) (layer "F.Cu") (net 10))
 (segment (start 107.5 59.52) (end 105.52 59.52) (width 0.25) (layer "F.Cu") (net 10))
 (segment (start 105.5 58) (end 106 57.5) (width 0.25) (layer "F.Cu") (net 10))
 (segment (start 106 59) (end 105.5 59.5) (width 0.25) (layer "F.Cu") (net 10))
 (segment (start 105.5 59.5) (end 105.5 58) (width 0.25) (layer "F.Cu") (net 10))
 (segment (start 115.52 59.52) (end 116 60) (width 0.25) (layer "F.Cu") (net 11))
 (segment (start 114 59.52) (end 115.52 59.52) (width 0.25) (layer "F.Cu") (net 11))
 (segment (start 116 59) (end 115 58) (width 0.25) (layer "F.Cu") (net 11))
 (segment (start 116 60) (end 116 59) (width 0.25) (layer "F.Cu") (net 11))
 (segment (start 112 57.88) (end 112 59.5) (width 0.5) (layer "F.Cu") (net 7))
 (segment (start 112.775 57.275) (end 114 58.5) (width 0.5) (layer "F.Cu") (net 7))
 (segment (start 112.775 57.105) (end 112 57.88) (width 0.5) (layer "F.Cu") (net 7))
 (segment (start 112.775 57.105) (end 112.775 57.275) (width 0.25) (layer "F.Cu") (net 7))
 (segment (start 113.2202 57.335) (end 112.775 57.335) (width 0.25) (layer "F.Cu") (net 7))
 (segment (start 114.435 54.565) (end 115.5 53.5) (width 0.25) (layer "F.Cu") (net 1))
 (segment (start 112.775 54.565) (end 114.435 54.565) (width 0.25) (layer "F.Cu") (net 1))
 (segment (start 115.335 55.835) (end 115.5 56) (width 0.25) (layer "F.Cu") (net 8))
 (segment (start 112.775 55.835) (end 115.335 55.835) (width 0.25) (layer "F.Cu") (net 8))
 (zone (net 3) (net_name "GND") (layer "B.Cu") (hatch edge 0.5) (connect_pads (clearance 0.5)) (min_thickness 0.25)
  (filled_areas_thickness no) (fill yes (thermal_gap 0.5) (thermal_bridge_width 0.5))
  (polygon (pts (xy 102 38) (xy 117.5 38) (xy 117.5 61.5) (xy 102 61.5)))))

